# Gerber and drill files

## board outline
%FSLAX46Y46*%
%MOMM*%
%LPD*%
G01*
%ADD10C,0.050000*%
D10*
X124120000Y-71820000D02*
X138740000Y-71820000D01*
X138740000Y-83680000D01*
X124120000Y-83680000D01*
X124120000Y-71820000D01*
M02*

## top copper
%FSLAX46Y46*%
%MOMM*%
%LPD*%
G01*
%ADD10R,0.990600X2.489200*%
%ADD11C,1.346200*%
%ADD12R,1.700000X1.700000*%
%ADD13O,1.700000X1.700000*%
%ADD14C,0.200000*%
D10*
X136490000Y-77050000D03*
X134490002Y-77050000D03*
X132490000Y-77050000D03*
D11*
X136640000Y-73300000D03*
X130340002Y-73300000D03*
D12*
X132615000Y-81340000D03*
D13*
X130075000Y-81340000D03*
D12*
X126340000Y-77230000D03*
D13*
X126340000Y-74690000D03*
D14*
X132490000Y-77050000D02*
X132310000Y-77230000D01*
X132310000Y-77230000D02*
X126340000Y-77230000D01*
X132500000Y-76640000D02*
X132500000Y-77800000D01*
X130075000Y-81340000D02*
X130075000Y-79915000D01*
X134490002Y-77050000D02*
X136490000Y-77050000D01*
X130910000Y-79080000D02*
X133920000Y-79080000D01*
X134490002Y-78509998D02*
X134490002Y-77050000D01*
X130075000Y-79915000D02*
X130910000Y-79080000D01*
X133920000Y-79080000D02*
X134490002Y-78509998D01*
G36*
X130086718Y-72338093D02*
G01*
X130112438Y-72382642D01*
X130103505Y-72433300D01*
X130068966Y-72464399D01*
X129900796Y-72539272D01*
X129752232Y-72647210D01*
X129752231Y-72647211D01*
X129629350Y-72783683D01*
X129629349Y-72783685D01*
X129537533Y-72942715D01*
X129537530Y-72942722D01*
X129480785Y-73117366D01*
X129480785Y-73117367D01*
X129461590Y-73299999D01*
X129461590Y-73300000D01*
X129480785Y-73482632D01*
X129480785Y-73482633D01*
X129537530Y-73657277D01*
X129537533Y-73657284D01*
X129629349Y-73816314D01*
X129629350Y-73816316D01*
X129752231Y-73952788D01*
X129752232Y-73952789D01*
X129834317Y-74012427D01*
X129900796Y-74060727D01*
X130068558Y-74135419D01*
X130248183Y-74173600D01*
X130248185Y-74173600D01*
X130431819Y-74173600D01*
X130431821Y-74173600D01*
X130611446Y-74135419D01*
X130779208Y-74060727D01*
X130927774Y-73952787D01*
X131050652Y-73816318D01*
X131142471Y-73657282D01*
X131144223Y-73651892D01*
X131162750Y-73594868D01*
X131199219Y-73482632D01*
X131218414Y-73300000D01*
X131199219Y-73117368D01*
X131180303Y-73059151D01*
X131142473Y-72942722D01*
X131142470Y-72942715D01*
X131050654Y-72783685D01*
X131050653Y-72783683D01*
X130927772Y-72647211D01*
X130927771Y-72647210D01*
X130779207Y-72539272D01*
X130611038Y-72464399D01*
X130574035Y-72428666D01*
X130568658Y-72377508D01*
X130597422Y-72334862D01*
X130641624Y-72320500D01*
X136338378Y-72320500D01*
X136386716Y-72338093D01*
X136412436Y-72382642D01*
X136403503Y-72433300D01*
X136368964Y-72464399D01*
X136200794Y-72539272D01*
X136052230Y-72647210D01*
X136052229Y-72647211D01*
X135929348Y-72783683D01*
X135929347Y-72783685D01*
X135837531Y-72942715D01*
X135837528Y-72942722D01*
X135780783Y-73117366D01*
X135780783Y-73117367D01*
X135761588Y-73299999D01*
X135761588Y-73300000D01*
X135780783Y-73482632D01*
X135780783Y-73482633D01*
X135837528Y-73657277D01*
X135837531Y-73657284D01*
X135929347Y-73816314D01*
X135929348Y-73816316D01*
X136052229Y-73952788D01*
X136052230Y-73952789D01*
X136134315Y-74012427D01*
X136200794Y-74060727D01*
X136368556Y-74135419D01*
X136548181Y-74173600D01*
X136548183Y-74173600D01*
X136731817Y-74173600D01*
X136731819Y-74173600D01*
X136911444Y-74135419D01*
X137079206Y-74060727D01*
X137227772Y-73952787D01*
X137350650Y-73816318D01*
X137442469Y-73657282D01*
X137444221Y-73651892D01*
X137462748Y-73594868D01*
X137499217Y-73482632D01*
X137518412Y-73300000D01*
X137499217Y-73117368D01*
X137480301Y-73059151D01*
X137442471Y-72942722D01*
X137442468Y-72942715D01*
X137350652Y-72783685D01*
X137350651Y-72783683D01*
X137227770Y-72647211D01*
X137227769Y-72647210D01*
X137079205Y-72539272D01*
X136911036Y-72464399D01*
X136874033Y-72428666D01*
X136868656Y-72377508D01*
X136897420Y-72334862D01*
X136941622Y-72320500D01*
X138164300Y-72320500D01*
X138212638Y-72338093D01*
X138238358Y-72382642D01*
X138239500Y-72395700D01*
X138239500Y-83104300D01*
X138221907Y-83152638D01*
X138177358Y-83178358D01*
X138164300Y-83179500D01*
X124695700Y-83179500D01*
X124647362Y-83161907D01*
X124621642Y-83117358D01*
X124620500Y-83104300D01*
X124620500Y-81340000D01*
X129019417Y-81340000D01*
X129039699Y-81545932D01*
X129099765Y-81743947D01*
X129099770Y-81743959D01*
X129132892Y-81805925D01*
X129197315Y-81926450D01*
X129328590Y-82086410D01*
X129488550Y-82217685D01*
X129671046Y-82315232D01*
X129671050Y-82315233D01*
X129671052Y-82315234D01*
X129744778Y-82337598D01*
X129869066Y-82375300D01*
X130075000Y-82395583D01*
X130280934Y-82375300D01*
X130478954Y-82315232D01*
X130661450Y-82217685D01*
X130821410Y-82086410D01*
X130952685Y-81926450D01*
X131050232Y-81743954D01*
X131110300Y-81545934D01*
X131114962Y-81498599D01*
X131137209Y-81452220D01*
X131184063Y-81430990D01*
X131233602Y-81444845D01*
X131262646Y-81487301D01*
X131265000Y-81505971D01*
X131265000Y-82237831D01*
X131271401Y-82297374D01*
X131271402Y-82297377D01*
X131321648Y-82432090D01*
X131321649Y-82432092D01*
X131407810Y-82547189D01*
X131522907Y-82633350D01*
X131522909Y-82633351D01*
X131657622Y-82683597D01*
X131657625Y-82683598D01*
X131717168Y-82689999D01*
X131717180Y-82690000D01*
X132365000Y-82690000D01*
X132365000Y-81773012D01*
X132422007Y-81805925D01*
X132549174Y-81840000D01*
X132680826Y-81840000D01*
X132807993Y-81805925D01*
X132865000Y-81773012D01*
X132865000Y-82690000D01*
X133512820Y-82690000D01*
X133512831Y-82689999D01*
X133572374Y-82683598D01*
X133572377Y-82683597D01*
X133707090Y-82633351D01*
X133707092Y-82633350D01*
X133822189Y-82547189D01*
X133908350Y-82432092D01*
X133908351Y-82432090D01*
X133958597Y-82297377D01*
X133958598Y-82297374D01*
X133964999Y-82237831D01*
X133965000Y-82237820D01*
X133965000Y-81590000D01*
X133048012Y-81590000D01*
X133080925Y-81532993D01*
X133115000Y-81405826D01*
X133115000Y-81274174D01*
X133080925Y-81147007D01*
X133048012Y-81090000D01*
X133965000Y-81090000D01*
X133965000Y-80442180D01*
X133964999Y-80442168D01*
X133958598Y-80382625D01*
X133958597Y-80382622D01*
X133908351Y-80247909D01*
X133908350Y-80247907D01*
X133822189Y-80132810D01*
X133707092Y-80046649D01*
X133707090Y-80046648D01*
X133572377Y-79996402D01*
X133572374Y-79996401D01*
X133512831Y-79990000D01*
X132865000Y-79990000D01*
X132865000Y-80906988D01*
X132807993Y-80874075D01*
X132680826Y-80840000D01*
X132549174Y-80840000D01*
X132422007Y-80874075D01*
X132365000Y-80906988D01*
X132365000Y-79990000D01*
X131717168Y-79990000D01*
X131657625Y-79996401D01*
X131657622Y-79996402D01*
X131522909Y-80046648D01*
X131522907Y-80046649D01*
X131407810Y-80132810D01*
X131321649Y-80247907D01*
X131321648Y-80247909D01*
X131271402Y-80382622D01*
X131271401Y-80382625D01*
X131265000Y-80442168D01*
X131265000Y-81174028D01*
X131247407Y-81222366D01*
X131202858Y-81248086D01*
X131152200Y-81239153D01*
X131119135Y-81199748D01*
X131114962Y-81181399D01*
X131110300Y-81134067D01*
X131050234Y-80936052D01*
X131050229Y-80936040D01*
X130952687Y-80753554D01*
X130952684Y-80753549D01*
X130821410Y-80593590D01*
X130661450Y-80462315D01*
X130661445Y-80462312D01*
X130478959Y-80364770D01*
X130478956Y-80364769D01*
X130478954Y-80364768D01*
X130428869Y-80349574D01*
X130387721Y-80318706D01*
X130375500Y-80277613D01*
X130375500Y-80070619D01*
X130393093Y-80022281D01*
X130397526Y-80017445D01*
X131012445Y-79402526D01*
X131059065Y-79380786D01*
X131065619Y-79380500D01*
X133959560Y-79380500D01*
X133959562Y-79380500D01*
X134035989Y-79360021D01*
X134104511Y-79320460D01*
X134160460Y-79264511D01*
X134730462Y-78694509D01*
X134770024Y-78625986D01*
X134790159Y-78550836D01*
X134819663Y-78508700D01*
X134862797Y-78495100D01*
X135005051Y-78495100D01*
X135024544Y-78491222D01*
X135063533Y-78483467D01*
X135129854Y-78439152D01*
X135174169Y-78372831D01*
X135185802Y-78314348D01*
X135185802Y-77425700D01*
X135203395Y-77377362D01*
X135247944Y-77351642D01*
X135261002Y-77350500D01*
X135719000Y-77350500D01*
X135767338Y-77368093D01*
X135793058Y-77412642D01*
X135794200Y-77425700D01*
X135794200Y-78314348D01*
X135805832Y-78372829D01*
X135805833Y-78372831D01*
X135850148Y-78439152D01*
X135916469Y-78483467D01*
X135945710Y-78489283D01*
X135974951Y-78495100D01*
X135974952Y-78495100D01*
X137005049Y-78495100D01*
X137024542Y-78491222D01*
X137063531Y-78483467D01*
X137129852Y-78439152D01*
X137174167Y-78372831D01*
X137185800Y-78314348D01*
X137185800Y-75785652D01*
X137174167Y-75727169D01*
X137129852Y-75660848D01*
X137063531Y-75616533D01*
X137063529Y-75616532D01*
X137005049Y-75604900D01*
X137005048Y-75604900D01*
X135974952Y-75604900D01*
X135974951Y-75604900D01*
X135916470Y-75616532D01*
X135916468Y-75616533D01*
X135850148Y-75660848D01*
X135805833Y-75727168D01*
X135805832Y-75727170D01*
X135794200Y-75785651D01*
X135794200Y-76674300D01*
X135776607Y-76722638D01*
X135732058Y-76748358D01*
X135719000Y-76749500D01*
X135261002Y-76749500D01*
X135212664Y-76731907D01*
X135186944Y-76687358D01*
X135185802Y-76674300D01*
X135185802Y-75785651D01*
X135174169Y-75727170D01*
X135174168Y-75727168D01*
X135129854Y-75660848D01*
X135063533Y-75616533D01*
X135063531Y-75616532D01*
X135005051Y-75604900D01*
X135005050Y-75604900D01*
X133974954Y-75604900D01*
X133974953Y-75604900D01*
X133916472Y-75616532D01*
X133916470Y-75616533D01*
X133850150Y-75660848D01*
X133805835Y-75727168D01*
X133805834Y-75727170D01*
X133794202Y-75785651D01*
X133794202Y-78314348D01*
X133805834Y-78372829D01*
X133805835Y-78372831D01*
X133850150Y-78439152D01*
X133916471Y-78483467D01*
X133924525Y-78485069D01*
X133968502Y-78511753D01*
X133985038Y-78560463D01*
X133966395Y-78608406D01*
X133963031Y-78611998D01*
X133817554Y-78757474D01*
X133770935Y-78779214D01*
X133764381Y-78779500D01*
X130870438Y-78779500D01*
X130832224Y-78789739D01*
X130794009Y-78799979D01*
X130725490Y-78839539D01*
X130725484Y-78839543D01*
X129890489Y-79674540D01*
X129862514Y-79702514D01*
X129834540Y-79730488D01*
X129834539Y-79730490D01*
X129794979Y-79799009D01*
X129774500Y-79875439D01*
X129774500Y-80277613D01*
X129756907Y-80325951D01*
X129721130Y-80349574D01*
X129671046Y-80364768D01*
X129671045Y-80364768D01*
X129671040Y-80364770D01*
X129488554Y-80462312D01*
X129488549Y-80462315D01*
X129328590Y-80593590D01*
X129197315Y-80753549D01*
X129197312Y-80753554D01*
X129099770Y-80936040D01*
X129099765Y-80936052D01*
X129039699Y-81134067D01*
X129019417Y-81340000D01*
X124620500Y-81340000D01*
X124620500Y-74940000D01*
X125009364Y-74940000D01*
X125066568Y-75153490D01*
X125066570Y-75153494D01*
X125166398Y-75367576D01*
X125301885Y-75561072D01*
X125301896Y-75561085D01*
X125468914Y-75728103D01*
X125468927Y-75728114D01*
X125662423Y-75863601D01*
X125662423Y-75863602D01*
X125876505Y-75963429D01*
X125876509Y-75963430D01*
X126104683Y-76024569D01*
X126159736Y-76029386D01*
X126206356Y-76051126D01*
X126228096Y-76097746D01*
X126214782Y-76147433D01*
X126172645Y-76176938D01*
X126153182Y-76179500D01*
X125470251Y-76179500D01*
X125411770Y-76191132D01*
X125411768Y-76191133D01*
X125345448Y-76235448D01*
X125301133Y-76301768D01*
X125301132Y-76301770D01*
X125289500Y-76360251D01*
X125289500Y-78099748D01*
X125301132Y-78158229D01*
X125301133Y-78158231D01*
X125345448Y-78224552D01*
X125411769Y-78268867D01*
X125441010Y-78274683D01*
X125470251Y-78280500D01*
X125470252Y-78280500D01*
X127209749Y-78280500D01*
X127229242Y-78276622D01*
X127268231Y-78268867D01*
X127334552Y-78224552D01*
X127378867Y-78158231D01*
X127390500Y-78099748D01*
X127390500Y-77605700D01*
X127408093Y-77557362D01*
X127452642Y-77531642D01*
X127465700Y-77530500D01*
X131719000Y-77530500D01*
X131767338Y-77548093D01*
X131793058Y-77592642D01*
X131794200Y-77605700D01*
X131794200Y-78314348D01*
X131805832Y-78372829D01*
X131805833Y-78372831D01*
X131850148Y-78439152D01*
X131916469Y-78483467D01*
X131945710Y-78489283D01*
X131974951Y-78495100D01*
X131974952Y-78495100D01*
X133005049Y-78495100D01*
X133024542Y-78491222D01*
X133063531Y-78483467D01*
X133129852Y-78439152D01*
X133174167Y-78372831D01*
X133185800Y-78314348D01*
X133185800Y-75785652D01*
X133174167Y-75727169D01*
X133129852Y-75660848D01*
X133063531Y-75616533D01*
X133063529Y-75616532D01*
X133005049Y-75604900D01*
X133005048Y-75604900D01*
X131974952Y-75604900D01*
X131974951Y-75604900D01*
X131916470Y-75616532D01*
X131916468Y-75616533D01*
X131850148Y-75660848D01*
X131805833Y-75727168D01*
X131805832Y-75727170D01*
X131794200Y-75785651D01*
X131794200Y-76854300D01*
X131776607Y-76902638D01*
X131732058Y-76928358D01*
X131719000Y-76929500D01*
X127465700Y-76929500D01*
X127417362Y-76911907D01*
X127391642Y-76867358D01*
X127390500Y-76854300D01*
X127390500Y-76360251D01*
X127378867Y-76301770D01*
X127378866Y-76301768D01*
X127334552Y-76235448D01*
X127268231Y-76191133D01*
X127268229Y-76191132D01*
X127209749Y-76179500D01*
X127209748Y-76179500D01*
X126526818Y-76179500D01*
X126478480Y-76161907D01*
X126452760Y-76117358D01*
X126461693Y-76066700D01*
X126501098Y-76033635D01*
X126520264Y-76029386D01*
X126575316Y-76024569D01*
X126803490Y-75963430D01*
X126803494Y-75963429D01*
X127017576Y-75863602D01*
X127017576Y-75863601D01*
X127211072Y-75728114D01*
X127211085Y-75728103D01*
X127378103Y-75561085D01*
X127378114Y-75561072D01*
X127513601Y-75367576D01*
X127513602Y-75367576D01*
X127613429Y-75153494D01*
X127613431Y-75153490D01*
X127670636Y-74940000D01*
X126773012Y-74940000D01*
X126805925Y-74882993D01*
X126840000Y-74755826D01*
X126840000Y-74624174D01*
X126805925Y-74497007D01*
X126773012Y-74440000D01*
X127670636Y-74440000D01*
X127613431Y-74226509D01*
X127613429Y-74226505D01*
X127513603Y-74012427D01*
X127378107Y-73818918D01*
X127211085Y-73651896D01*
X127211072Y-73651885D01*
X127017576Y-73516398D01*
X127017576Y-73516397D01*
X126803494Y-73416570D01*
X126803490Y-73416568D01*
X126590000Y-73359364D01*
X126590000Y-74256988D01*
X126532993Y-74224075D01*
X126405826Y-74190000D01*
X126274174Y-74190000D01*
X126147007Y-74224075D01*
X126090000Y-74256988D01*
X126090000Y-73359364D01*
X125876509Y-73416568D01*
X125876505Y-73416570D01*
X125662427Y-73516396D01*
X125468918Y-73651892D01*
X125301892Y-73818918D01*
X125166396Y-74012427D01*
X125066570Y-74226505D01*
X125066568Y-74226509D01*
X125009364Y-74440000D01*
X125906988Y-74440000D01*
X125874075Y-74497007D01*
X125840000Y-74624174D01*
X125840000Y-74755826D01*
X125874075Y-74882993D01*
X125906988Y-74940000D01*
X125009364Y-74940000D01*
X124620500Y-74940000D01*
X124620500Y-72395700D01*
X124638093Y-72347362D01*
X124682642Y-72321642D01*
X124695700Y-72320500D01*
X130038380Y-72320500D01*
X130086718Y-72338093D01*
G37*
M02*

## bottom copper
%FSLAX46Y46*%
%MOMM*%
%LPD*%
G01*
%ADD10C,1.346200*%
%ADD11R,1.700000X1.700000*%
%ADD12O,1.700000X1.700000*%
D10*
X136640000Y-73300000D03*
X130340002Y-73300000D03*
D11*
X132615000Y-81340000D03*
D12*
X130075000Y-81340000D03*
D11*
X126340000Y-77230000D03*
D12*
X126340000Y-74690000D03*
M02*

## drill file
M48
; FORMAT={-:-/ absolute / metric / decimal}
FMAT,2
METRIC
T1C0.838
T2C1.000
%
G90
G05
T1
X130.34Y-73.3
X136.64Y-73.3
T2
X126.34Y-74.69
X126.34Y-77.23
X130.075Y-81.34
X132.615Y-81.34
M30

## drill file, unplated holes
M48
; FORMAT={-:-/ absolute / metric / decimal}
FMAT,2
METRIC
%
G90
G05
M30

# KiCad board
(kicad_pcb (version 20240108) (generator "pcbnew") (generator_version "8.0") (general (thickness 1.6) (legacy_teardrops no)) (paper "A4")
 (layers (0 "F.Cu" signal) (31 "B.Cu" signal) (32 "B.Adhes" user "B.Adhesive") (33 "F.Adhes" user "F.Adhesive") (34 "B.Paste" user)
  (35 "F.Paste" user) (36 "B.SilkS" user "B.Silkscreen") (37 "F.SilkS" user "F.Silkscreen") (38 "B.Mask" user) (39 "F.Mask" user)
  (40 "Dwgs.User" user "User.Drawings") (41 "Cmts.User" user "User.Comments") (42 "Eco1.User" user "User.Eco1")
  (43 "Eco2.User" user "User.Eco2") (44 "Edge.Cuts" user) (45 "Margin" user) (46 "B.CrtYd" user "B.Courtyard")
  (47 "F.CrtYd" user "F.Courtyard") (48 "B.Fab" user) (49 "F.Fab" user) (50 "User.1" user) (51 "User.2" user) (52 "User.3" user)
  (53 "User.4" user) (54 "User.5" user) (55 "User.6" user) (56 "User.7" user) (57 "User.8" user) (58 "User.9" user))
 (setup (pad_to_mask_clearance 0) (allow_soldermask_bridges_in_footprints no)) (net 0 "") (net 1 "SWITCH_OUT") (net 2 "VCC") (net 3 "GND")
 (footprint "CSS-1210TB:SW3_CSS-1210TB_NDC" (layer "F.Cu") (at 133.490001 73.704287 180)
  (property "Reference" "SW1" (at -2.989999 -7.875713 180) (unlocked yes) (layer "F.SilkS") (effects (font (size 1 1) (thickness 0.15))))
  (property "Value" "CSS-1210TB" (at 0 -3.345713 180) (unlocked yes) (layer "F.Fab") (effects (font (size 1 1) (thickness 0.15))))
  (pad "1" smd rect (at -2.999999 -3.345713 180) (size 0.9906 2.4892) (layers "F.Cu" "F.Paste" "F.Mask") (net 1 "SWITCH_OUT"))
  (pad "2" smd rect (at -1.000001 -3.345713 180) (size 0.9906 2.4892) (layers "F.Cu" "F.Paste" "F.Mask") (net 1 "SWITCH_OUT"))
  (pad "3" smd rect (at 1.000001 -3.345713 180) (size 0.9906 2.4892) (layers "F.Cu" "F.Paste" "F.Mask") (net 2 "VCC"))
  (pad "5" thru_hole circle (at -3.149999 0.404287 180) (size 1.3462 1.3462) (drill 0.8382) (layers "*.Cu" "*.Mask")
   (remove_unused_layers no))
  (pad "6" thru_hole circle (at 3.149999 0.404287 180) (size 1.3462 1.3462) (drill 0.8382) (layers "*.Cu" "*.Mask")
   (remove_unused_layers no)))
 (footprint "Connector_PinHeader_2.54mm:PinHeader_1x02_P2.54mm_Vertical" (layer "F.Cu") (at 132.615 81.34 -90)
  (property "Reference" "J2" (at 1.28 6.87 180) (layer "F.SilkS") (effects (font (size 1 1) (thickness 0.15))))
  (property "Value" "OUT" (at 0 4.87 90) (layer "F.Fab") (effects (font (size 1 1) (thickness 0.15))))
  (pad "1" thru_hole rect (at 0 0 270) (size 1.7 1.7) (drill 1) (layers "*.Cu" "*.Mask") (remove_unused_layers no) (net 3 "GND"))
  (pad "2" thru_hole oval (at 0 2.54 270) (size 1.7 1.7) (drill 1) (layers "*.Cu" "*.Mask") (remove_unused_layers no) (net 1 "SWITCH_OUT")))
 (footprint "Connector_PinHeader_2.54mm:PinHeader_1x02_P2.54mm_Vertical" (layer "B.Cu") (at 126.34 77.23)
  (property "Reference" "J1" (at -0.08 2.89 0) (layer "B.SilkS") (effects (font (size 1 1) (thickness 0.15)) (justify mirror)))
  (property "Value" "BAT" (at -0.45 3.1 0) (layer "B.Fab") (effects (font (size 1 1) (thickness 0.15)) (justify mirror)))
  (pad "1" thru_hole rect (at 0 0) (size 1.7 1.7) (drill 1) (layers "*.Cu" "*.Mask") (remove_unused_layers no) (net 2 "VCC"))
  (pad "2" thru_hole oval (at 0 -2.54) (size 1.7 1.7) (drill 1) (layers "*.Cu" "*.Mask") (remove_unused_layers no) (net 3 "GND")))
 (gr_rect (start 124.12 71.82) (end 138.74 83.68) (stroke (width 0.05) (type default)) (fill none) (layer "Edge.Cuts"))
 (segment (start 132.49 77.05) (end 132.31 77.23) (width 0.2) (layer "F.Cu") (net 2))
 (segment (start 132.31 77.23) (end 126.34 77.23) (width 0.2) (layer "F.Cu") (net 2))
 (segment (start 132.5 76.64) (end 132.5 77.8) (width 0.2) (layer "F.Cu") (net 2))
 (segment (start 130.075 81.34) (end 130.075 79.915) (width 0.2) (layer "F.Cu") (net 1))
 (segment (start 134.490002 77.05) (end 136.49 77.05) (width 0.2) (layer "F.Cu") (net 1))
 (segment (start 130.91 79.08) (end 133.92 79.08) (width 0.2) (layer "F.Cu") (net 1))
 (segment (start 134.490002 78.509998) (end 134.490002 77.05) (width 0.2) (layer "F.Cu") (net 1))
 (segment (start 130.075 79.915) (end 130.91 79.08) (width 0.2) (layer "F.Cu") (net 1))
 (segment (start 133.92 79.08) (end 134.490002 78.509998) (width 0.2) (layer "F.Cu") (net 1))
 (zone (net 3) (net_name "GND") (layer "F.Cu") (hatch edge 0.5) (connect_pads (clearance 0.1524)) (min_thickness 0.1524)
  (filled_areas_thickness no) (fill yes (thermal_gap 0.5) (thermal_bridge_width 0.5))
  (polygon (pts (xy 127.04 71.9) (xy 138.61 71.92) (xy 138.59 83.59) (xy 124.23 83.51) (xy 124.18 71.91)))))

